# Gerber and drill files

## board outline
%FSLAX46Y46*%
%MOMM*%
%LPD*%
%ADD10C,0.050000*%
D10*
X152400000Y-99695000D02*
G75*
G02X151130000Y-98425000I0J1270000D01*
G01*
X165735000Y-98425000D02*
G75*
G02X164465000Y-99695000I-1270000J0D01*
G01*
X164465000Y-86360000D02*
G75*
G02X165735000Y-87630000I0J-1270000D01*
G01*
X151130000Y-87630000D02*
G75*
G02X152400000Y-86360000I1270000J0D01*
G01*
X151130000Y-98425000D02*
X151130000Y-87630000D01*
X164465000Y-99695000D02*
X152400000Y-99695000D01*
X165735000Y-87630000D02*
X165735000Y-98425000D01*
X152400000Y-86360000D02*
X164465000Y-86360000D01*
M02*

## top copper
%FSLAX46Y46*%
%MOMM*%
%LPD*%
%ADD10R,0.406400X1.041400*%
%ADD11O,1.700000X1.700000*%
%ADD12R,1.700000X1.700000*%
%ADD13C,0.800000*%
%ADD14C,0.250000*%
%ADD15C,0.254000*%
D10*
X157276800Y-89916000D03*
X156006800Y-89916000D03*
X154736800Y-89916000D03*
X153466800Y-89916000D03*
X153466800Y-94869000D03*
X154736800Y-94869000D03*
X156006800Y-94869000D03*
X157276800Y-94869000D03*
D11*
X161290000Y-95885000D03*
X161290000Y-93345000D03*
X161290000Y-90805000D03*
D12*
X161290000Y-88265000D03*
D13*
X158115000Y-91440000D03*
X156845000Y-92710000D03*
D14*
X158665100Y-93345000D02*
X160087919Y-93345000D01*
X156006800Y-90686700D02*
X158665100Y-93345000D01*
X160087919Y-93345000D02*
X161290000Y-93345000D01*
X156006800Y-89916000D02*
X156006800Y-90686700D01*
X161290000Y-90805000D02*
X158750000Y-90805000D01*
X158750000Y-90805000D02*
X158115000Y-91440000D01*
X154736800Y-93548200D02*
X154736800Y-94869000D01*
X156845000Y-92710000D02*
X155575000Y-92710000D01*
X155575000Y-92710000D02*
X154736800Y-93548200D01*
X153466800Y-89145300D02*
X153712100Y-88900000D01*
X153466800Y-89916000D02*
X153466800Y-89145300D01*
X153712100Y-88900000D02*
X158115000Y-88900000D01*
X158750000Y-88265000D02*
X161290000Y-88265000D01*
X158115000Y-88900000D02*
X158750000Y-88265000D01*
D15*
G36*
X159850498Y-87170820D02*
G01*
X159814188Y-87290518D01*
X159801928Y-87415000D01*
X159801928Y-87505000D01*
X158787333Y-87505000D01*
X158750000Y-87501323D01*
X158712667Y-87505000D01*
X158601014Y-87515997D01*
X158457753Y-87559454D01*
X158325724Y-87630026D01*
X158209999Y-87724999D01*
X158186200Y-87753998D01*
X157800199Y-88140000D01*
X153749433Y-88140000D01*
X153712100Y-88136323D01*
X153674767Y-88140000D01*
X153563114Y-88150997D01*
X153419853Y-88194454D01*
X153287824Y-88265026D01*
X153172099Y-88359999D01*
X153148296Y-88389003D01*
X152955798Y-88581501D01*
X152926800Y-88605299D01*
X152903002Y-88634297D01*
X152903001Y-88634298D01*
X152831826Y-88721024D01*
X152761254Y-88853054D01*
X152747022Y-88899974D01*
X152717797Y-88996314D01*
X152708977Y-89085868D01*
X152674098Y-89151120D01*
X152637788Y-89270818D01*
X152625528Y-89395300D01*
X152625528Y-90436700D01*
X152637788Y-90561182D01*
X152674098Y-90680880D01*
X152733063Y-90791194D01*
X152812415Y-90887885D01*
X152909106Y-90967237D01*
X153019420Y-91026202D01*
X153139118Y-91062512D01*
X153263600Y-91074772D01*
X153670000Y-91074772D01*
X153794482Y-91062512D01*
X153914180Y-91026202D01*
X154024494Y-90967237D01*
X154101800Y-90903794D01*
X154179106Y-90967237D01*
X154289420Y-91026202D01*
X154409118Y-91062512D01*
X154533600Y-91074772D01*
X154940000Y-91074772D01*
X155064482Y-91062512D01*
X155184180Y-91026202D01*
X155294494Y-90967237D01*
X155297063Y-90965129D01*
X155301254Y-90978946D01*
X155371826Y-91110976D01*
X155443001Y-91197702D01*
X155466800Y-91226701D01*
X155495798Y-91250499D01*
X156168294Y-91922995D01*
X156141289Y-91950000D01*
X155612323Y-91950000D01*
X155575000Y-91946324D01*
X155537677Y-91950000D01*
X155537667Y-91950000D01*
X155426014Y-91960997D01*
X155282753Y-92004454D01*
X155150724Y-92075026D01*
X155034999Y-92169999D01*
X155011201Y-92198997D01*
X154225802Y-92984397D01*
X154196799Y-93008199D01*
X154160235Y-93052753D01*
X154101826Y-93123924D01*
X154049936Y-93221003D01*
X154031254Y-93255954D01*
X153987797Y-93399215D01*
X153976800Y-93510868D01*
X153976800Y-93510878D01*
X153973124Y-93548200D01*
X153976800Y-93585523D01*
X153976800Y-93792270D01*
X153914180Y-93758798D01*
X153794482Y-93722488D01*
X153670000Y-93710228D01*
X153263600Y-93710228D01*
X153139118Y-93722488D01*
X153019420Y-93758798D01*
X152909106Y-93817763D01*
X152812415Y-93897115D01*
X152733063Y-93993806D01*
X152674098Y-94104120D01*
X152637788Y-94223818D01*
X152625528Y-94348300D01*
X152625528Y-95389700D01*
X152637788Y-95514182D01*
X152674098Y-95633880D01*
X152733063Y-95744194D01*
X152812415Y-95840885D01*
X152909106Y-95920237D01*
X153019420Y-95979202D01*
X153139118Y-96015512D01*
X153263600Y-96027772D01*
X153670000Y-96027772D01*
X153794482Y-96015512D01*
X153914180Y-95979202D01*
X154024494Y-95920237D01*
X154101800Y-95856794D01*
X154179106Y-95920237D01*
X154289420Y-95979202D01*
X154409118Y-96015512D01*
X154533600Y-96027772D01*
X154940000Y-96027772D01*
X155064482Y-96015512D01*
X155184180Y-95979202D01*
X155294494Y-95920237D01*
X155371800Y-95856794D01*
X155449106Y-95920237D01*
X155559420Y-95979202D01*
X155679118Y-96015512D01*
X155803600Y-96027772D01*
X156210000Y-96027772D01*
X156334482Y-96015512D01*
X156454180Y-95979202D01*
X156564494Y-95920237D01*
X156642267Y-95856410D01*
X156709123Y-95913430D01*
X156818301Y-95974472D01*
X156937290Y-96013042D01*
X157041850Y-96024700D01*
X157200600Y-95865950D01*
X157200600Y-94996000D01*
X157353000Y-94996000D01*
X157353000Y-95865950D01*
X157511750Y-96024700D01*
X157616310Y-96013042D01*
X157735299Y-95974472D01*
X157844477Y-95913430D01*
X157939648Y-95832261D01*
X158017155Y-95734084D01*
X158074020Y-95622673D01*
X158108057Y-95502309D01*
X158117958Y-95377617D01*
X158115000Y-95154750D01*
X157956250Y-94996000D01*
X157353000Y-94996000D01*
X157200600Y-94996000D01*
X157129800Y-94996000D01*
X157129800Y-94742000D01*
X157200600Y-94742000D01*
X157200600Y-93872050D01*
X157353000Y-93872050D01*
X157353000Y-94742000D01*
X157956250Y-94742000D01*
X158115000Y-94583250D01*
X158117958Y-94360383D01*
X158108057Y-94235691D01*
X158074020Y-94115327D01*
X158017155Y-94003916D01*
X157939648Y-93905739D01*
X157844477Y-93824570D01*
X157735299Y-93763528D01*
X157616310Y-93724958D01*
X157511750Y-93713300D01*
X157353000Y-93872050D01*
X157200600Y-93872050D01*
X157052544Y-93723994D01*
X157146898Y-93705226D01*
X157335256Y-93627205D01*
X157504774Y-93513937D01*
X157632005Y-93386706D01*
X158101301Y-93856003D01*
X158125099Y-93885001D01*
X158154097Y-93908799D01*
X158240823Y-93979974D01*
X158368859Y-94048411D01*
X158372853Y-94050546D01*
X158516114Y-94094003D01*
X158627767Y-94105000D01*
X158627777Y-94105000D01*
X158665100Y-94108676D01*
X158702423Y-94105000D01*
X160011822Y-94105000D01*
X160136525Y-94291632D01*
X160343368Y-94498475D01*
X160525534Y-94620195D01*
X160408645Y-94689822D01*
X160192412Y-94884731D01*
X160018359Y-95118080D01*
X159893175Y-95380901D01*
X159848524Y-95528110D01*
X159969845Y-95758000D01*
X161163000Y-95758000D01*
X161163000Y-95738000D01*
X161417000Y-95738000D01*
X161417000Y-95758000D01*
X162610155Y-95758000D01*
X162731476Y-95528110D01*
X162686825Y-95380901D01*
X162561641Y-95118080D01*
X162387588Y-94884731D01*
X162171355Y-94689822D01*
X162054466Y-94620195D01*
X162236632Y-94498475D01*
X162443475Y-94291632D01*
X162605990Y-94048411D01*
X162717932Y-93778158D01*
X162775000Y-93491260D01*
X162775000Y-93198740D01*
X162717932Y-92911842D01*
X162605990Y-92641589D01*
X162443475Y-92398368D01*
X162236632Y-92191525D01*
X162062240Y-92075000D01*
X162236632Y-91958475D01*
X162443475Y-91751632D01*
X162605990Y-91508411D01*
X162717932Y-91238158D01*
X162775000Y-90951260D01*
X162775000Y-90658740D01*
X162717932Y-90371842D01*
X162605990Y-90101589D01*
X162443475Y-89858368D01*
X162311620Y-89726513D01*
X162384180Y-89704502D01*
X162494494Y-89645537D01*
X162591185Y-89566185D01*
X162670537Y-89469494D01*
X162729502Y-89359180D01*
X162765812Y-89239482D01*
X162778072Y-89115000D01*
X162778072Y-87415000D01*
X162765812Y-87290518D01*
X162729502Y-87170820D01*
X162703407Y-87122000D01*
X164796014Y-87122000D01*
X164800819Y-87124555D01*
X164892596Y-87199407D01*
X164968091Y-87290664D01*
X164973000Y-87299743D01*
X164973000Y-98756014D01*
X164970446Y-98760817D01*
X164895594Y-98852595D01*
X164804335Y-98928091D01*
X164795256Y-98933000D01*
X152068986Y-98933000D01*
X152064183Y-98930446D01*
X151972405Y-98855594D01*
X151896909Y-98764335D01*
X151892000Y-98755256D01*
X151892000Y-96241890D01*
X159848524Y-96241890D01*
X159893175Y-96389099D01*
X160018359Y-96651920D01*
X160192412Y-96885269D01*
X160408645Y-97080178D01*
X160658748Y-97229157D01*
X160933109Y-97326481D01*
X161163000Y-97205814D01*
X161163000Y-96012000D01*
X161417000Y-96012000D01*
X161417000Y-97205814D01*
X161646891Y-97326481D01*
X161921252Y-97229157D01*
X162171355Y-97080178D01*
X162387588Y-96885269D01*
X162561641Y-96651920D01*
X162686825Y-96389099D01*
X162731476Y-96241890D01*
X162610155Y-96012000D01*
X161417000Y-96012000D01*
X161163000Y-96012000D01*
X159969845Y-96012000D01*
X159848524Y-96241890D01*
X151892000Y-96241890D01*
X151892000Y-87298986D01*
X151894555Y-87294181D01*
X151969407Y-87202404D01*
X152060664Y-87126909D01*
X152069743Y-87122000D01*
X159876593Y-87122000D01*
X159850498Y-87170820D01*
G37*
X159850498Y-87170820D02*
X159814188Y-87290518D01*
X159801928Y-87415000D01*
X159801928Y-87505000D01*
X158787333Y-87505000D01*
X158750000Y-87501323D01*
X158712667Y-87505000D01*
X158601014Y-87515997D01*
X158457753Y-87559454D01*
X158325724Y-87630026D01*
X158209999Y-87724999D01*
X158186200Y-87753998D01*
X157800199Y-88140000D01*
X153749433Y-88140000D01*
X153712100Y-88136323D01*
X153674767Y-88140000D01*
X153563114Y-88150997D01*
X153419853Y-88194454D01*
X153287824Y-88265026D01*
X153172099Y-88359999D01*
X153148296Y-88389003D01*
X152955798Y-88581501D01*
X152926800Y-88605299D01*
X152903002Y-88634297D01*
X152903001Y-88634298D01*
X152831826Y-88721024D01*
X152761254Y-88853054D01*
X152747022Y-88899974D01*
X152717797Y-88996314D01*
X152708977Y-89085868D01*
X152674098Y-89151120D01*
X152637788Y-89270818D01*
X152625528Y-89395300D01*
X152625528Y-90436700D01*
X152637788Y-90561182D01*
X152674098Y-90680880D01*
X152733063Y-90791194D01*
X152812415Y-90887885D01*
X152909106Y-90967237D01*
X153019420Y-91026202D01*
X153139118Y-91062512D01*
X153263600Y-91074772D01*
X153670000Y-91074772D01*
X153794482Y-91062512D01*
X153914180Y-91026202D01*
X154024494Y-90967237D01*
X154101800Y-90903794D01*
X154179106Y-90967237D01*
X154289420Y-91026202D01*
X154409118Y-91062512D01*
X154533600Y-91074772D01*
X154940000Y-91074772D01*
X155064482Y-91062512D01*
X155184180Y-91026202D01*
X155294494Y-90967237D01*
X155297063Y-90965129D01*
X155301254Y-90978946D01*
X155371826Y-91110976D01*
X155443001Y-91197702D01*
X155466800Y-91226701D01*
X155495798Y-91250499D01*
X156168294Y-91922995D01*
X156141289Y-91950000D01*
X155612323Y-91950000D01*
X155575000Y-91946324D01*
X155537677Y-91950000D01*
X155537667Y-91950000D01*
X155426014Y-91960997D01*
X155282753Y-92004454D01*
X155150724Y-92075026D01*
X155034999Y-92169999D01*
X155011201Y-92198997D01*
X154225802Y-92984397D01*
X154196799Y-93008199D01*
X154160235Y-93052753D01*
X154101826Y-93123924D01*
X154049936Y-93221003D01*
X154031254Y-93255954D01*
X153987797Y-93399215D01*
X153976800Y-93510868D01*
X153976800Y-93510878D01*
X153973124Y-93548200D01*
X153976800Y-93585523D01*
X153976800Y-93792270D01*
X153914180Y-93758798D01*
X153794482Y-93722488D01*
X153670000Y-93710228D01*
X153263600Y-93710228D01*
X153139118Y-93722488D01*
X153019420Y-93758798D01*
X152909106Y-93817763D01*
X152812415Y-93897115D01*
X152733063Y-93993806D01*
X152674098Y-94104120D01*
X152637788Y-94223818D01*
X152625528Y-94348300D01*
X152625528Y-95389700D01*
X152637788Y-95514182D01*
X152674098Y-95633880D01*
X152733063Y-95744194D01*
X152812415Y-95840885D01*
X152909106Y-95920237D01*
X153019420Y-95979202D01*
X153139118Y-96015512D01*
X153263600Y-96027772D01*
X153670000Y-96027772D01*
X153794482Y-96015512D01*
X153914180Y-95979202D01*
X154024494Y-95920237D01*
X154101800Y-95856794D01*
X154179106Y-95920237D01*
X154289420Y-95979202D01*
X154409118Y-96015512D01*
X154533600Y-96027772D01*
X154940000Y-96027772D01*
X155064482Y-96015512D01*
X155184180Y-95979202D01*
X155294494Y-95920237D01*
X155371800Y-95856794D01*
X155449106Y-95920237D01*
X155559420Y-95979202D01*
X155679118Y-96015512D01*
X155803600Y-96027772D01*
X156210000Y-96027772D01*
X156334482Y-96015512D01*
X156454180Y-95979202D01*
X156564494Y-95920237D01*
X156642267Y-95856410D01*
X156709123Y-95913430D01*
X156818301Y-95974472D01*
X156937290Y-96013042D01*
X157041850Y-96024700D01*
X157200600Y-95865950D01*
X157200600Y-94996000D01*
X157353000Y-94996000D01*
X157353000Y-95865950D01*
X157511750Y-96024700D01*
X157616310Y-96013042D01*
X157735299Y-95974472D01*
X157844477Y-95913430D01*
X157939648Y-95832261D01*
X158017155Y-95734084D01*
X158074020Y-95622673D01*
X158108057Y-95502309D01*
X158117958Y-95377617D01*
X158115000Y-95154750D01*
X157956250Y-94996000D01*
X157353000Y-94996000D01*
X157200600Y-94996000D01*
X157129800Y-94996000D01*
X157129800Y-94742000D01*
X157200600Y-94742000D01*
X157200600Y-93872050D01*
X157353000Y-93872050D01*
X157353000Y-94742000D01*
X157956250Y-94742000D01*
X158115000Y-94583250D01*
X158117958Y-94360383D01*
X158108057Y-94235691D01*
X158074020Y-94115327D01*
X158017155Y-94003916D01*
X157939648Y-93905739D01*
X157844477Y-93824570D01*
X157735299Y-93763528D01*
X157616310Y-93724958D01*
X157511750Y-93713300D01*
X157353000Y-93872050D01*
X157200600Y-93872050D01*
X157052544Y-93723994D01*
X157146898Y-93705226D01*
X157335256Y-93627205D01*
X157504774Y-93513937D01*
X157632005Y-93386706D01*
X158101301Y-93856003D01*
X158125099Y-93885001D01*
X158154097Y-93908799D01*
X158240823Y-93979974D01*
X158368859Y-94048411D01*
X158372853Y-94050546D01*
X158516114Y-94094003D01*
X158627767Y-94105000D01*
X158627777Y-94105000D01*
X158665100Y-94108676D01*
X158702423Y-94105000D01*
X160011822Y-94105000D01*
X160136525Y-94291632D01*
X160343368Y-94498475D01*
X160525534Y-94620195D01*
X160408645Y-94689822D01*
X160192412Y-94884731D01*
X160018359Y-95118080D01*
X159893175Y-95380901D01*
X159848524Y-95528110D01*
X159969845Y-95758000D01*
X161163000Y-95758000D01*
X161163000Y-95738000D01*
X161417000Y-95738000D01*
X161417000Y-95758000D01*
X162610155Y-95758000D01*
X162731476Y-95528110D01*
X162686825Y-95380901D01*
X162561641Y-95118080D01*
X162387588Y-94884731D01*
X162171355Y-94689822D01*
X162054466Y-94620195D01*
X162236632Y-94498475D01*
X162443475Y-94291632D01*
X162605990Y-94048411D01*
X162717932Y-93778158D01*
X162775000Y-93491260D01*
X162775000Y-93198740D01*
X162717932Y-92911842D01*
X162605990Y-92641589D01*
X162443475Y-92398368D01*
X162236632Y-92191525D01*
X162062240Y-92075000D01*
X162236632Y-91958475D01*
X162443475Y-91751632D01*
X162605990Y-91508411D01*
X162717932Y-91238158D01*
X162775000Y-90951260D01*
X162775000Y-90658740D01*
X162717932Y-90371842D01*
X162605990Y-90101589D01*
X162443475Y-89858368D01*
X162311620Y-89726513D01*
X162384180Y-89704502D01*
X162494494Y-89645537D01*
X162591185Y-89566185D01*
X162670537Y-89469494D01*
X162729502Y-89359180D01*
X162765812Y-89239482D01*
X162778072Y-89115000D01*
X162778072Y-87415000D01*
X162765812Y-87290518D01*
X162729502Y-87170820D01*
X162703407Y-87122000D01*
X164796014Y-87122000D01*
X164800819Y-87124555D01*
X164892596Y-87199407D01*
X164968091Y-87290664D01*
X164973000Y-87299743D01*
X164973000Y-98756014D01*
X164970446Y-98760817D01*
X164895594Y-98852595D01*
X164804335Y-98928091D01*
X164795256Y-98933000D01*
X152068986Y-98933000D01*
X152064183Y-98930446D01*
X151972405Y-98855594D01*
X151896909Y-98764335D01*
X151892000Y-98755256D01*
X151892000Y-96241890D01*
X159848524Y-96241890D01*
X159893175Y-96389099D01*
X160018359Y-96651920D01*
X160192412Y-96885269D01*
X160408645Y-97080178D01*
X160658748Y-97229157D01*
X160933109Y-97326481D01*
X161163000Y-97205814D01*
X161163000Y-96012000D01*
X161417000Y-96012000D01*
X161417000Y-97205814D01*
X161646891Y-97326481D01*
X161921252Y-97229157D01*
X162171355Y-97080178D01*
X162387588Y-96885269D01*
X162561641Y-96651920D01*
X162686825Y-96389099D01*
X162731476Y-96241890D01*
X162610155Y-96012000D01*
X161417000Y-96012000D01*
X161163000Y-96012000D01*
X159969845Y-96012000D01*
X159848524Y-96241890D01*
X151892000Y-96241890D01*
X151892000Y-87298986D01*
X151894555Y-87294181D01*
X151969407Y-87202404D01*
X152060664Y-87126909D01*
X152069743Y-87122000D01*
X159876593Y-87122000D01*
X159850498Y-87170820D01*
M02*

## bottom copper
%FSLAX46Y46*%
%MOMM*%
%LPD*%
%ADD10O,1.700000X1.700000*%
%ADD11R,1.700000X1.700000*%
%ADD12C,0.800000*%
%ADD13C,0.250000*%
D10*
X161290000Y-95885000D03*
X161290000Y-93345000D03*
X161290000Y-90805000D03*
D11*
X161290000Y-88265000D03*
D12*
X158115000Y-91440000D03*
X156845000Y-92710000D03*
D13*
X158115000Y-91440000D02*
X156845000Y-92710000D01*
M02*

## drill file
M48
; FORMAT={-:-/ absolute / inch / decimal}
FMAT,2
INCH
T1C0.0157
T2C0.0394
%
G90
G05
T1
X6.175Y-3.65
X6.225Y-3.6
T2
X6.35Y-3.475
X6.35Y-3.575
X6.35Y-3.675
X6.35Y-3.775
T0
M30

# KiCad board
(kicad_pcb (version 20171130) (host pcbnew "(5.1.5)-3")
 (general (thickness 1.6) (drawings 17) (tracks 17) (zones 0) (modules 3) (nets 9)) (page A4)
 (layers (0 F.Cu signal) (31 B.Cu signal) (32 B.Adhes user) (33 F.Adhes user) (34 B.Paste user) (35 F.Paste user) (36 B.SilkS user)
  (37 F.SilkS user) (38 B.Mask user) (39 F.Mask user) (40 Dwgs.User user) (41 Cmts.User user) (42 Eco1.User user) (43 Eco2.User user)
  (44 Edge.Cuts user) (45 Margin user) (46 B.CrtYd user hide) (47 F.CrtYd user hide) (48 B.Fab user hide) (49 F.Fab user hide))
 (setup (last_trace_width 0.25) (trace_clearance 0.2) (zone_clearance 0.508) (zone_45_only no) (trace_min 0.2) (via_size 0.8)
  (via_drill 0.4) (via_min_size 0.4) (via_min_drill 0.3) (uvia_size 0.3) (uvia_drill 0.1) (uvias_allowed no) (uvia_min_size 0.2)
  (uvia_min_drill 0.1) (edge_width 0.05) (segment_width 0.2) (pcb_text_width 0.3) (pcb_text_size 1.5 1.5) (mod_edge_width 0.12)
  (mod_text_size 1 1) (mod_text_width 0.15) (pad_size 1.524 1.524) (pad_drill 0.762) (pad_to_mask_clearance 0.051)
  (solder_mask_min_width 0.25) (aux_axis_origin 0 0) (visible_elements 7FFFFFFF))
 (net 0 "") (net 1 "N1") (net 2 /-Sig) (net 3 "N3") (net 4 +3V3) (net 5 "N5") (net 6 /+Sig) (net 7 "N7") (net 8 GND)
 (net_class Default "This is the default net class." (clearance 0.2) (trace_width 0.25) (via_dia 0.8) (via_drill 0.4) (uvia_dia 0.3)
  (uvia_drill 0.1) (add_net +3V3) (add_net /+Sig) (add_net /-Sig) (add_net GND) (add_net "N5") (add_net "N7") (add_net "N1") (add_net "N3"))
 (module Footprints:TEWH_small (layer B.Cu) (at 155.575 91.44 180)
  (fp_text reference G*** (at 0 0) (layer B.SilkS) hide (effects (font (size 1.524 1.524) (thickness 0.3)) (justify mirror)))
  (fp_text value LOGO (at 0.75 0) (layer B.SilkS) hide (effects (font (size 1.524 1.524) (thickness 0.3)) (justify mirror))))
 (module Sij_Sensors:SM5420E (layer F.Cu) (at 160.02 92.075 90)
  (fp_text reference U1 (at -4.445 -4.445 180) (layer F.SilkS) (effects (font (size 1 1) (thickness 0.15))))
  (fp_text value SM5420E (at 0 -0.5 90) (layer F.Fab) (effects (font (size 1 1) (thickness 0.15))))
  (pad 5 smd rect (at 2.159 -2.7432 90) (size 1.0414 0.4064) (layers F.Cu F.Paste F.Mask) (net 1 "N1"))
  (pad 6 smd rect (at 2.159 -4.0132 90) (size 1.0414 0.4064) (layers F.Cu F.Paste F.Mask) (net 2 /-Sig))
  (pad 7 smd rect (at 2.159 -5.2832 90) (size 1.0414 0.4064) (layers F.Cu F.Paste F.Mask) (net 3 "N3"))
  (pad 8 smd rect (at 2.159 -6.5532 90) (size 1.0414 0.4064) (layers F.Cu F.Paste F.Mask) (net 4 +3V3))
  (pad 1 smd rect (at -2.794 -6.5532 90) (size 1.0414 0.4064) (layers F.Cu F.Paste F.Mask) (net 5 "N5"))
  (pad 2 smd rect (at -2.794 -5.2832 90) (size 1.0414 0.4064) (layers F.Cu F.Paste F.Mask) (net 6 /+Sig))
  (pad 3 smd rect (at -2.794 -4.0132 90) (size 1.0414 0.4064) (layers F.Cu F.Paste F.Mask) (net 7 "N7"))
  (pad 4 smd rect (at -2.794 -2.7432 90) (size 1.0414 0.4064) (layers F.Cu F.Paste F.Mask) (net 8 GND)))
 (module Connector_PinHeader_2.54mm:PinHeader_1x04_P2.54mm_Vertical (layer B.Cu) (at 161.29 88.265 180)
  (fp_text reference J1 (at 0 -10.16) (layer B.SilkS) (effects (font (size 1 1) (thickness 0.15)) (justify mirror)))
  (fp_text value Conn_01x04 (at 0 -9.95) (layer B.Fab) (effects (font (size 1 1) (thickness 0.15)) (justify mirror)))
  (pad 4 thru_hole oval (at 0 -7.62 180) (size 1.7 1.7) (drill 1) (layers *.Cu *.Mask) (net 8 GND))
  (pad 3 thru_hole oval (at 0 -5.08 180) (size 1.7 1.7) (drill 1) (layers *.Cu *.Mask) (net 2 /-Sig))
  (pad 2 thru_hole oval (at 0 -2.54 180) (size 1.7 1.7) (drill 1) (layers *.Cu *.Mask) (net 6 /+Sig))
  (pad 1 thru_hole rect (at 0 0 180) (size 1.7 1.7) (drill 1) (layers *.Cu *.Mask) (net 4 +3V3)))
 (gr_arc (start 152.4 98.425) (end 151.13 98.425) (angle -90) (layer Edge.Cuts) (width 0.05))
 (gr_arc (start 164.465 98.425) (end 164.465 99.695) (angle -90) (layer Edge.Cuts) (width 0.05))
 (gr_arc (start 164.465 87.63) (end 165.735 87.63) (angle -90) (layer Edge.Cuts) (width 0.05))
 (gr_arc (start 152.4 87.63) (end 152.4 86.36) (angle -90) (layer Edge.Cuts) (width 0.05))
 (gr_line (start 151.13 98.425) (end 151.13 87.63) (layer Edge.Cuts) (width 0.05))
 (gr_line (start 164.465 99.695) (end 152.4 99.695) (layer Edge.Cuts) (width 0.05))
 (gr_line (start 165.735 87.63) (end 165.735 98.425) (layer Edge.Cuts) (width 0.05))
 (gr_line (start 152.4 86.36) (end 164.465 86.36) (layer Edge.Cuts) (width 0.05))
 (segment (start 158.6651 93.345) (end 160.087919 93.345) (width 0.25) (layer F.Cu) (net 2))
 (segment (start 156.0068 90.6867) (end 158.6651 93.345) (width 0.25) (layer F.Cu) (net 2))
 (segment (start 160.087919 93.345) (end 161.29 93.345) (width 0.25) (layer F.Cu) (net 2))
 (segment (start 156.0068 89.916) (end 156.0068 90.6867) (width 0.25) (layer F.Cu) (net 2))
 (via (at 158.115 91.44) (size 0.8) (drill 0.4) (layers F.Cu B.Cu) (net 6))
 (segment (start 161.29 90.805) (end 158.75 90.805) (width 0.25) (layer F.Cu) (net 6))
 (segment (start 158.75 90.805) (end 158.115 91.44) (width 0.25) (layer F.Cu) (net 6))
 (via (at 156.845 92.71) (size 0.8) (drill 0.4) (layers F.Cu B.Cu) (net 6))
 (segment (start 158.115 91.44) (end 156.845 92.71) (width 0.25) (layer B.Cu) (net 6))
 (segment (start 154.7368 93.5482) (end 154.7368 94.869) (width 0.25) (layer F.Cu) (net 6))
 (segment (start 156.845 92.71) (end 155.575 92.71) (width 0.25) (layer F.Cu) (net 6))
 (segment (start 155.575 92.71) (end 154.7368 93.5482) (width 0.25) (layer F.Cu) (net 6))
 (segment (start 153.4668 89.1453) (end 153.7121 88.9) (width 0.25) (layer F.Cu) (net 4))
 (segment (start 153.4668 89.916) (end 153.4668 89.1453) (width 0.25) (layer F.Cu) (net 4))
 (segment (start 153.7121 88.9) (end 158.115 88.9) (width 0.25) (layer F.Cu) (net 4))
 (segment (start 158.75 88.265) (end 161.29 88.265) (width 0.25) (layer F.Cu) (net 4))
 (segment (start 158.115 88.9) (end 158.75 88.265) (width 0.25) (layer F.Cu) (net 4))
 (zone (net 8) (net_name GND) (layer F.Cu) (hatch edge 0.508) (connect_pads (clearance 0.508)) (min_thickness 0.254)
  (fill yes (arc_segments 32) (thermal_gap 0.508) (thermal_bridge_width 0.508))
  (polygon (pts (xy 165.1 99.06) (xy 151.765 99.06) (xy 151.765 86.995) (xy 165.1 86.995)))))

